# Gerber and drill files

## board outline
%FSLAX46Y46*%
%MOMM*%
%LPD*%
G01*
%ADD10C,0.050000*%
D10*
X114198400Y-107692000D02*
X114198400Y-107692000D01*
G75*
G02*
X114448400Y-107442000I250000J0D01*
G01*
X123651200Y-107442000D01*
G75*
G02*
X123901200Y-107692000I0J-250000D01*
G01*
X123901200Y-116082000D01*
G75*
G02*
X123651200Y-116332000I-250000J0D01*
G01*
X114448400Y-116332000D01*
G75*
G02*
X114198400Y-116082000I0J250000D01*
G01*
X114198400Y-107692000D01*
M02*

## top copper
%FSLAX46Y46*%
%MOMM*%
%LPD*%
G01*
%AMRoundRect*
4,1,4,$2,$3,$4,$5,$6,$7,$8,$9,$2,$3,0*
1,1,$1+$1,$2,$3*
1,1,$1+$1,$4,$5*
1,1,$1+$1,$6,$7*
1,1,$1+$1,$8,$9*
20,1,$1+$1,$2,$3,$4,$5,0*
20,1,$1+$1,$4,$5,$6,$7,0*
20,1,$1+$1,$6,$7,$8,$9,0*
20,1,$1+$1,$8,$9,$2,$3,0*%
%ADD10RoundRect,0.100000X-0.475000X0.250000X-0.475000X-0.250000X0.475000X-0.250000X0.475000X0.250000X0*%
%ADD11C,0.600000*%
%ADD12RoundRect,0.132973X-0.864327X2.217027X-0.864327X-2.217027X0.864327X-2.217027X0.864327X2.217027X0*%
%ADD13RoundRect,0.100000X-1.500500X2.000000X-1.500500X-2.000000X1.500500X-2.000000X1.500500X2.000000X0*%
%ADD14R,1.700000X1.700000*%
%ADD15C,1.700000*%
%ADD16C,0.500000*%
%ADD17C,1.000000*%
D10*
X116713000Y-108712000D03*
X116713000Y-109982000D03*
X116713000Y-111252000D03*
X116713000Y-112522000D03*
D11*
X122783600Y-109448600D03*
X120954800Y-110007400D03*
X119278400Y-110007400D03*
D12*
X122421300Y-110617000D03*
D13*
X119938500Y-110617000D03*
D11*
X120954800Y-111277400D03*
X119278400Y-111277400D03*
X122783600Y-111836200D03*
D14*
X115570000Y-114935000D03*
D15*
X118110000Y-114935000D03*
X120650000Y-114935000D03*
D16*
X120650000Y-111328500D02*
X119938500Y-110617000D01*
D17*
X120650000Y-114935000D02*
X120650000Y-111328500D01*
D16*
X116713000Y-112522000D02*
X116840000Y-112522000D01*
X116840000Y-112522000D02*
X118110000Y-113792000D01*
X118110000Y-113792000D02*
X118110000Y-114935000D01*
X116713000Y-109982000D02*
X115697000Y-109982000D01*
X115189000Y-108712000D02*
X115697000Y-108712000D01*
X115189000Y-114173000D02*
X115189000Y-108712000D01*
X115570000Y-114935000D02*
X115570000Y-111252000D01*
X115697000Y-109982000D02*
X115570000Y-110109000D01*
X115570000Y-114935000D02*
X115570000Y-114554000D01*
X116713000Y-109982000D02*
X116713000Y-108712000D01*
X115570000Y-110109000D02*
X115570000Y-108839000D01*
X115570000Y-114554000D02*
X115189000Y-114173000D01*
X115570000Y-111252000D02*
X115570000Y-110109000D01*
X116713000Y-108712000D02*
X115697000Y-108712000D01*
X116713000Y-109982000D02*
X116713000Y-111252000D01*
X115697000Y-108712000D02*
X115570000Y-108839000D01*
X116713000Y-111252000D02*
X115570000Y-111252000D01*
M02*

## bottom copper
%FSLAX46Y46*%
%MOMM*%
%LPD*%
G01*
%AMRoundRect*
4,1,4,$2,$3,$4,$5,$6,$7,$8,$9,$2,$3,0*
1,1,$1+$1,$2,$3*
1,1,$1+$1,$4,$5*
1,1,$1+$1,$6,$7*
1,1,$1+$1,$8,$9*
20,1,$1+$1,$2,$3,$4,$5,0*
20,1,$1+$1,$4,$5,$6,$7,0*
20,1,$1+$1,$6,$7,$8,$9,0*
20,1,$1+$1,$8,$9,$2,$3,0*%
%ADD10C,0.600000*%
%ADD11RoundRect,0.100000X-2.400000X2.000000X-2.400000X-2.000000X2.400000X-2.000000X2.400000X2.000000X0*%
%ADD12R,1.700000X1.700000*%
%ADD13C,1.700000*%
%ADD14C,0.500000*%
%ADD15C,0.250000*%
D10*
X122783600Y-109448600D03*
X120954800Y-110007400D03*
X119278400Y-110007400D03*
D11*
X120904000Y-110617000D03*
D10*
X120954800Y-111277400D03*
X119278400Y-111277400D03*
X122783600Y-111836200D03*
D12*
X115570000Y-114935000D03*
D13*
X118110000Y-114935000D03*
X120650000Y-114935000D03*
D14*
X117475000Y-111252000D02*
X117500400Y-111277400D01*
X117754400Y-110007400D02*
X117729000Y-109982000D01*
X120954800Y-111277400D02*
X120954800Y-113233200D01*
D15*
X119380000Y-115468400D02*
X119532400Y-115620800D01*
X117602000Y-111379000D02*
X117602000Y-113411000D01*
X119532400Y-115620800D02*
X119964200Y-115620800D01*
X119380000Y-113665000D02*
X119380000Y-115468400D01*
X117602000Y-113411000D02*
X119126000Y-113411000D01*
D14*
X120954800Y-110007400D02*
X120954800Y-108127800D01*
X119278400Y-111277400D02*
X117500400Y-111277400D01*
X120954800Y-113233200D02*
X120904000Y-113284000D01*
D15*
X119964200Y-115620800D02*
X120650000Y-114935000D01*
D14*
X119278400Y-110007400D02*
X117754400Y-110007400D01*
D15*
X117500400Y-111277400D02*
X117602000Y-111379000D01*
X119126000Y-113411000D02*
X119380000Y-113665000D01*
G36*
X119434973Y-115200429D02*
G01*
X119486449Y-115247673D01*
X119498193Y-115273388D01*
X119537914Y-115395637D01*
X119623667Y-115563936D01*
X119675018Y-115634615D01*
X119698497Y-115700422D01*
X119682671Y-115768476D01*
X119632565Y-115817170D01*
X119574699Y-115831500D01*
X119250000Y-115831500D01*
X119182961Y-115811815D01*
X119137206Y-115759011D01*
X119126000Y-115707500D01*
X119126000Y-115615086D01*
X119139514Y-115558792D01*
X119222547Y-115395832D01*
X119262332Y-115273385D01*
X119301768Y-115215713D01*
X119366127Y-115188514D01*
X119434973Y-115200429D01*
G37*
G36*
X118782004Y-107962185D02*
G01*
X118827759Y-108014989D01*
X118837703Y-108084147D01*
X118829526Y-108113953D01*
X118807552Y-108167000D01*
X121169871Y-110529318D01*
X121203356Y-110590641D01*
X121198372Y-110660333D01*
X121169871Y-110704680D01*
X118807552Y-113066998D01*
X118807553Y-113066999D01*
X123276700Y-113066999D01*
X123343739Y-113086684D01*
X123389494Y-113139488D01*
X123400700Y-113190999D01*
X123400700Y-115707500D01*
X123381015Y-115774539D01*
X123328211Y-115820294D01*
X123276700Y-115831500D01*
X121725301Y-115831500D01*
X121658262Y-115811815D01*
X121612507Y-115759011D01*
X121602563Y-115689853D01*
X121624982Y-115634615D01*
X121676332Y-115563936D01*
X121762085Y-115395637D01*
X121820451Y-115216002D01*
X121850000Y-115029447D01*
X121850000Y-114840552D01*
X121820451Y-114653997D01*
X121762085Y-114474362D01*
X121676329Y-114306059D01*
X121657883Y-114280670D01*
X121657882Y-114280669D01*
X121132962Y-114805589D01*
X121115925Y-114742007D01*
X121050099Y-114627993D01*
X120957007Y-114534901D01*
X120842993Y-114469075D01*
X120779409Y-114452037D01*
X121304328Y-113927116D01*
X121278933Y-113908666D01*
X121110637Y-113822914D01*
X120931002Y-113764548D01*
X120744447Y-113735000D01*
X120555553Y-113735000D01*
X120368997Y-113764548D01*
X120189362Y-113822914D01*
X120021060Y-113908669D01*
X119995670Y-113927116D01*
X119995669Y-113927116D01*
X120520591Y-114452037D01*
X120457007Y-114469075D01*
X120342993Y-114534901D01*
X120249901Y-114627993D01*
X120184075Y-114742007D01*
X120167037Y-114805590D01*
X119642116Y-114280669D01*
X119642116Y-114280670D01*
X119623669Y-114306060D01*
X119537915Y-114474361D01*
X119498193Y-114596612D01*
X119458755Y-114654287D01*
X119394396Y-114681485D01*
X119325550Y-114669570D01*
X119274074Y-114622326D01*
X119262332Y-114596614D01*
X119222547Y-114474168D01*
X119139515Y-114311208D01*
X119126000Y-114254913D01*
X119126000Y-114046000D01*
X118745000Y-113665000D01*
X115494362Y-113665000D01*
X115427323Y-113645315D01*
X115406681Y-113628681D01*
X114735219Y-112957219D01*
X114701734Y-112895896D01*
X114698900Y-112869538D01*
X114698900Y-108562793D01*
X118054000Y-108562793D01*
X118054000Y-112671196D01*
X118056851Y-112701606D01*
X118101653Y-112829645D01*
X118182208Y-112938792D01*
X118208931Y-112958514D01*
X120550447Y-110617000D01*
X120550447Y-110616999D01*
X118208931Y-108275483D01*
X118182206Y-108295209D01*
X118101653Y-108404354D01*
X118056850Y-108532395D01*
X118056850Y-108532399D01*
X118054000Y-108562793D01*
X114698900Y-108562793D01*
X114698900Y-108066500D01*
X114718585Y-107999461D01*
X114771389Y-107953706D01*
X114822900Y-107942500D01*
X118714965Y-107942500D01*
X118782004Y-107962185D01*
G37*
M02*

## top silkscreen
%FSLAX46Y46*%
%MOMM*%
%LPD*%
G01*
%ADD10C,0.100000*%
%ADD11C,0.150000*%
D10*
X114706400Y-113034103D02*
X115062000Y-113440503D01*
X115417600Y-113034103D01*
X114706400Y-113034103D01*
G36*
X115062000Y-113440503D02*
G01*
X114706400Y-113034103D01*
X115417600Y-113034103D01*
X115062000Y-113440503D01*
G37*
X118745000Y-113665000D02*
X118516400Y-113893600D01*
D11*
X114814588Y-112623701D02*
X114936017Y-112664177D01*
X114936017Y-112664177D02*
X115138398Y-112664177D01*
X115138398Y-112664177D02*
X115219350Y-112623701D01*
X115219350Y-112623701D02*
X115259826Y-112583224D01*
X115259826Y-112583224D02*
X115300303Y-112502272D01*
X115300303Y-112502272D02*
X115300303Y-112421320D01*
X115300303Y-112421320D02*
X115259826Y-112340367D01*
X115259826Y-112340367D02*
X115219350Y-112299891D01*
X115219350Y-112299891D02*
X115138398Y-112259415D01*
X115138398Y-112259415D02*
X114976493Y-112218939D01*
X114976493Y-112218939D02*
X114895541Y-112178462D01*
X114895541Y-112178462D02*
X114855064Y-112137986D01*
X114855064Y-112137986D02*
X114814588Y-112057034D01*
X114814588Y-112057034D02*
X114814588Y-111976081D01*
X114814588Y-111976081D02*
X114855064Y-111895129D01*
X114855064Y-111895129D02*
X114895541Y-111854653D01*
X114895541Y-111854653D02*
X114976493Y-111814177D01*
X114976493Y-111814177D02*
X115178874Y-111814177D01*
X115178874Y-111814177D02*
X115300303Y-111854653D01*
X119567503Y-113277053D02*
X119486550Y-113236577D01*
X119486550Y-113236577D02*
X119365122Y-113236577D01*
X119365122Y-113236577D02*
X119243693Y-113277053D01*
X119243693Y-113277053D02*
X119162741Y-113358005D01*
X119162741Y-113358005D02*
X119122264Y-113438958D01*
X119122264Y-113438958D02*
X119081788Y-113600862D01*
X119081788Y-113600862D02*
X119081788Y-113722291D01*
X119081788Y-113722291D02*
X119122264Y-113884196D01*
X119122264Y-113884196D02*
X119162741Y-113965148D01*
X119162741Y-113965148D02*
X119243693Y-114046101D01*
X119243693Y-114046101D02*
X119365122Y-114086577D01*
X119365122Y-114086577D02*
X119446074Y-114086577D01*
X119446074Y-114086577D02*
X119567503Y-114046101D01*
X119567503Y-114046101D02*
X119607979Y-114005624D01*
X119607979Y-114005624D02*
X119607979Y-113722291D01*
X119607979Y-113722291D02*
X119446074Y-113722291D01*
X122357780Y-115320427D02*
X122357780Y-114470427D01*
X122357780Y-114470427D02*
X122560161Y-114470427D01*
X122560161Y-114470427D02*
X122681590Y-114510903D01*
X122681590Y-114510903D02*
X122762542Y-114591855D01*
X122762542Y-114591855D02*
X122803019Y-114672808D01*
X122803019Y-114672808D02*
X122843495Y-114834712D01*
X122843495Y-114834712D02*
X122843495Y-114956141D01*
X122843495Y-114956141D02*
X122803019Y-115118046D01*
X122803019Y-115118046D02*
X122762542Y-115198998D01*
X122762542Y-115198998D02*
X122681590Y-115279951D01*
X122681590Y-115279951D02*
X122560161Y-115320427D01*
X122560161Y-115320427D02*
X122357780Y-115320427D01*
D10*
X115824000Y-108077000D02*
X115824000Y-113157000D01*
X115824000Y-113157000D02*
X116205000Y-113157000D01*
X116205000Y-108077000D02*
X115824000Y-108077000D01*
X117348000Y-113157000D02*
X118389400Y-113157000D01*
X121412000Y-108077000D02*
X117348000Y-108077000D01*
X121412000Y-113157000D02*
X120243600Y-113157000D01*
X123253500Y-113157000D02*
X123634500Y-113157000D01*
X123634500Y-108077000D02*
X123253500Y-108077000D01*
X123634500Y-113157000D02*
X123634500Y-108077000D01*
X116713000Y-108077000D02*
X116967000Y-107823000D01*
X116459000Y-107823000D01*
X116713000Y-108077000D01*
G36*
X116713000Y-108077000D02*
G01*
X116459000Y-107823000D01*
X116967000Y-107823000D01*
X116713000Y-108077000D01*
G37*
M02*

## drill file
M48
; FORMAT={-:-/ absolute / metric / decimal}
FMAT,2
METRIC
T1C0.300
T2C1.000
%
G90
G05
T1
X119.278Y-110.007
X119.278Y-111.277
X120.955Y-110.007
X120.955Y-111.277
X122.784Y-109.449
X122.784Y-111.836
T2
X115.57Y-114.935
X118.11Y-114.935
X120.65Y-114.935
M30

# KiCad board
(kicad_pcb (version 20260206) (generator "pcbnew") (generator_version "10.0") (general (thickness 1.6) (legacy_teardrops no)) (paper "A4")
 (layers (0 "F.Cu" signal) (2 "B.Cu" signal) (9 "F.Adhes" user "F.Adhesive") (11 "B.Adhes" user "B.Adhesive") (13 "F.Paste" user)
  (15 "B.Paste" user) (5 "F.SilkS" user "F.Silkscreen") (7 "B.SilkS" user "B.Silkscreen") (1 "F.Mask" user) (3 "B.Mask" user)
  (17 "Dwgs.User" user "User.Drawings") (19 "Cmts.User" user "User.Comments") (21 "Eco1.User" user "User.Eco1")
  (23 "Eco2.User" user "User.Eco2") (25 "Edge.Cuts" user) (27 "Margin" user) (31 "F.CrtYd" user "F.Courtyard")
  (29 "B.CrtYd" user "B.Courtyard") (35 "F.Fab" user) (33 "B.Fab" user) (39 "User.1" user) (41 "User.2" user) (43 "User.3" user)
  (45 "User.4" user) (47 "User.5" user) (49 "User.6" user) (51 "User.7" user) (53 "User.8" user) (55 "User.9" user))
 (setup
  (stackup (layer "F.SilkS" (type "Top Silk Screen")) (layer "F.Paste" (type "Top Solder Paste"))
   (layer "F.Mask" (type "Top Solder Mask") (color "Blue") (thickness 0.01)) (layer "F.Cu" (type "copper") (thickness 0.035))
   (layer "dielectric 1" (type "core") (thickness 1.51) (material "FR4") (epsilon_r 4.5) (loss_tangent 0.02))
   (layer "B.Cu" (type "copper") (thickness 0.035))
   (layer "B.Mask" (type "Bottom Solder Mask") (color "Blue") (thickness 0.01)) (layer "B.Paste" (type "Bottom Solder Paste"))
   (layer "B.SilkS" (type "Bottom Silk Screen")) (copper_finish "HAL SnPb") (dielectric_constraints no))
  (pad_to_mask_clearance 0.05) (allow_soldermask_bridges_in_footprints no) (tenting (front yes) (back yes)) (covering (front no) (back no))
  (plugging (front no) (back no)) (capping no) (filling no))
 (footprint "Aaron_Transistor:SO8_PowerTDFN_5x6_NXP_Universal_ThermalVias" (layer "F.Cu") (at 122.936 110.617 -90)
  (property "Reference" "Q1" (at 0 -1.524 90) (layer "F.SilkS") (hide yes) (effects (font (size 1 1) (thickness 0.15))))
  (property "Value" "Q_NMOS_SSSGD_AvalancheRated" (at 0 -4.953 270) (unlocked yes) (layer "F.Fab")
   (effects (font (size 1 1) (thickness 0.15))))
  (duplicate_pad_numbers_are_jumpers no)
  (fp_line (start -2.54 7.112) (end 2.54 7.112) (stroke (width 0.1) (type default)) (layer "F.SilkS"))
  (fp_line (start 2.54 7.112) (end 2.54 6.731) (stroke (width 0.1) (type default)) (layer "F.SilkS"))
  (fp_line (start -2.54 6.731) (end -2.54 7.112) (stroke (width 0.1) (type default)) (layer "F.SilkS"))
  (fp_line (start 2.54 5.588) (end 2.54 4.5466) (stroke (width 0.1) (type default)) (layer "F.SilkS"))
  (fp_line (start -2.54 1.524) (end -2.54 5.588) (stroke (width 0.1) (type default)) (layer "F.SilkS"))
  (fp_line (start 2.54 1.524) (end 2.54 2.6924) (stroke (width 0.1) (type default)) (layer "F.SilkS"))
  (fp_line (start 2.54 -0.3175) (end 2.54 -0.6985) (stroke (width 0.1) (type default)) (layer "F.SilkS"))
  (fp_line (start -2.54 -0.6985) (end -2.54 -0.3175) (stroke (width 0.1) (type default)) (layer "F.SilkS"))
  (fp_line (start 2.54 -0.6985) (end -2.54 -0.6985) (stroke (width 0.1) (type default)) (layer "F.SilkS"))
  (fp_poly (pts (xy -2.54 6.223) (xy -2.794 5.969) (xy -2.794 6.477)) (stroke (width 0.1) (type solid)) (fill yes) (layer "F.SilkS"))
  (pad "1" smd roundrect (at -1.905 6.223 270) (size 0.7 1.15) (layers "F.Cu" "F.Mask" "F.Paste") (roundrect_rratio 0.1428571429)
   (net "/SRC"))
  (pad "2" smd roundrect (at -0.635 6.223 270) (size 0.7 1.15) (layers "F.Cu" "F.Mask" "F.Paste") (roundrect_rratio 0.1428571429)
   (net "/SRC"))
  (pad "3" smd roundrect (at 0.635 6.223 270) (size 0.7 1.15) (layers "F.Cu" "F.Mask" "F.Paste") (roundrect_rratio 0.1428571429)
   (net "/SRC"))
  (pad "4" smd roundrect (at 1.905 6.223 270) (size 0.7 1.15) (layers "F.Cu" "F.Mask" "F.Paste") (roundrect_rratio 0.1428571429)
   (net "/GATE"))
  (pad "5" thru_hole circle (at -1.1684 0.1524 270) (size 0.6 0.6) (drill 0.3) (layers "*.Cu" "*.Mask") (remove_unused_layers no)
   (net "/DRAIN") (zone_connect 2))
  (pad "5" thru_hole circle (at -0.6096 1.9812 270) (size 0.6 0.6) (drill 0.3) (layers "*.Cu" "*.Mask") (remove_unused_layers no)
   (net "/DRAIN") (zone_connect 2))
  (pad "5" thru_hole circle (at -0.6096 3.6576 270) (size 0.6 0.6) (drill 0.3) (layers "*.Cu" "*.Mask") (remove_unused_layers no)
   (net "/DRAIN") (zone_connect 2))
  (pad "5" smd roundrect (at 0 0.5147 270) (size 4.7 1.9946) (layers "F.Cu" "F.Mask") (roundrect_rratio 0.06666666667) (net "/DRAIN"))
  (pad "5" smd roundrect (at 0 2.032 270) (size 4.2 5) (layers "B.Cu" "B.Mask") (roundrect_rratio 0.02380952381) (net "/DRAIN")
   (thermal_bridge_angle 45))
  (pad "5" smd roundrect (at 0 2.9975 270) (size 4.2 3.201) (layers "F.Cu" "F.Mask") (roundrect_rratio 0.03124023743) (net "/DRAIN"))
  (pad "5" thru_hole circle (at 0.6604 1.9812 270) (size 0.6 0.6) (drill 0.3) (layers "*.Cu" "*.Mask") (remove_unused_layers no)
   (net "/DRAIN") (zone_connect 2))
  (pad "5" thru_hole circle (at 0.6604 3.6576 270) (size 0.6 0.6) (drill 0.3) (layers "*.Cu" "*.Mask") (remove_unused_layers no)
   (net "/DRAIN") (zone_connect 2))
  (pad "5" thru_hole circle (at 1.2192 0.1524 270) (size 0.6 0.6) (drill 0.3) (layers "*.Cu" "*.Mask") (remove_unused_layers no)
   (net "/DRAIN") (zone_connect 2)))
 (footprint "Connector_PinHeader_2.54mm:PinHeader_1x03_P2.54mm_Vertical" (layer "B.Cu") (at 115.57 114.935 -90)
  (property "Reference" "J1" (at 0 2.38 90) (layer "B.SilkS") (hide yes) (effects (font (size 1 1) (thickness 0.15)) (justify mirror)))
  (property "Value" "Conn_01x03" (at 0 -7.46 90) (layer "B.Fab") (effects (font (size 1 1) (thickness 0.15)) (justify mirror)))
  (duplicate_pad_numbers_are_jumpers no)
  (pad "1" thru_hole rect (at 0 0 270) (size 1.7 1.7) (drill 1) (layers "*.Cu" "*.Mask") (remove_unused_layers no) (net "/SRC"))
  (pad "2" thru_hole circle (at 0 -2.54 270) (size 1.7 1.7) (drill 1) (layers "*.Cu" "*.Mask") (remove_unused_layers no) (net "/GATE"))
  (pad "3" thru_hole circle (at 0 -5.08 270) (size 1.7 1.7) (drill 1) (layers "*.Cu" "*.Mask") (remove_unused_layers no) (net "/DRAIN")))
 (gr_poly
  (pts (xy 114.7064 113.034103) (xy 115.062 113.440503) (xy 115.4176 113.034103)) (stroke (width 0.1) (type solid)) (fill yes)
  (layer "F.SilkS"))
 (gr_line (start 118.745 113.665) (end 118.5164 113.8936) (stroke (width 0.1) (type default)) (layer "F.SilkS"))
 (gr_rect (start 114.1984 107.442) (end 123.9012 116.332) (radius 0.25) (stroke (width 0.05) (type solid)) (fill no) (layer "Edge.Cuts"))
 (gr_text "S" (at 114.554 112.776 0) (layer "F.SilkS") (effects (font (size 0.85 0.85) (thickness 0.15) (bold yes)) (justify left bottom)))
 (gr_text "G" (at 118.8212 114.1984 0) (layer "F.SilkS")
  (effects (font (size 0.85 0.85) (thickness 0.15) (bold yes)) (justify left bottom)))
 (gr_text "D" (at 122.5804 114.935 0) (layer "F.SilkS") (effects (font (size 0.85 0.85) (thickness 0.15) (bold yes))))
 (segment (start 120.65 111.3285) (end 119.9385 110.617) (width 0.5) (layer "F.Cu") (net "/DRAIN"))
 (segment (start 120.65 114.935) (end 120.65 111.3285) (width 1) (layer "F.Cu") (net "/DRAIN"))
 (segment (start 117.475 111.252) (end 117.5004 111.2774) (width 0.5) (layer "B.Cu") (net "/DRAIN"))
 (segment (start 117.7544 110.0074) (end 117.729 109.982) (width 0.5) (layer "B.Cu") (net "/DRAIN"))
 (segment (start 120.9548 111.2774) (end 120.9548 113.2332) (width 0.5) (layer "B.Cu") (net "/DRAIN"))
 (segment (start 119.38 115.4684) (end 119.5324 115.6208) (width 0.25) (layer "B.Cu") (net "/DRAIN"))
 (segment (start 117.602 111.379) (end 117.602 113.411) (width 0.25) (layer "B.Cu") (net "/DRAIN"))
 (segment (start 119.5324 115.6208) (end 119.9642 115.6208) (width 0.25) (layer "B.Cu") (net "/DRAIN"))
 (segment (start 119.38 113.665) (end 119.38 115.4684) (width 0.25) (layer "B.Cu") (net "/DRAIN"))
 (segment (start 117.602 113.411) (end 119.126 113.411) (width 0.25) (layer "B.Cu") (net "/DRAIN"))
 (segment (start 120.9548 110.0074) (end 120.9548 108.1278) (width 0.5) (layer "B.Cu") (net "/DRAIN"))
 (segment (start 119.2784 111.2774) (end 117.5004 111.2774) (width 0.5) (layer "B.Cu") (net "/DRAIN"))
 (segment (start 120.9548 113.2332) (end 120.904 113.284) (width 0.5) (layer "B.Cu") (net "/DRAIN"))
 (segment (start 119.9642 115.6208) (end 120.65 114.935) (width 0.25) (layer "B.Cu") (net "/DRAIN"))
 (segment (start 119.2784 110.0074) (end 117.7544 110.0074) (width 0.5) (layer "B.Cu") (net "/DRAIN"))
 (segment (start 117.5004 111.2774) (end 117.602 111.379) (width 0.25) (layer "B.Cu") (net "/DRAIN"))
 (segment (start 119.126 113.411) (end 119.38 113.665) (width 0.25) (layer "B.Cu") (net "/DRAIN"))
 (segment (start 116.713 112.522) (end 116.84 112.522) (width 0.5) (layer "F.Cu") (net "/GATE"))
 (segment (start 116.84 112.522) (end 118.11 113.792) (width 0.5) (layer "F.Cu") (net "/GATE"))
 (segment (start 118.11 113.792) (end 118.11 114.935) (width 0.5) (layer "F.Cu") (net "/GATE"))
 (segment (start 116.713 109.982) (end 115.697 109.982) (width 0.5) (layer "F.Cu") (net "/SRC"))
 (segment (start 115.189 108.712) (end 115.697 108.712) (width 0.5) (layer "F.Cu") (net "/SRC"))
 (segment (start 115.189 114.173) (end 115.189 108.712) (width 0.5) (layer "F.Cu") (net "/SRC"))
 (segment (start 115.57 114.935) (end 115.57 111.252) (width 0.5) (layer "F.Cu") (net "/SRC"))
 (segment (start 115.697 109.982) (end 115.57 110.109) (width 0.5) (layer "F.Cu") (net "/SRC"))
 (segment (start 115.57 114.935) (end 115.57 114.554) (width 0.5) (layer "F.Cu") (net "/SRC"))
 (segment (start 116.713 109.982) (end 116.713 108.712) (width 0.5) (layer "F.Cu") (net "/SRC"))
 (segment (start 115.57 110.109) (end 115.57 108.839) (width 0.5) (layer "F.Cu") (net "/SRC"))
 (segment (start 115.57 114.554) (end 115.189 114.173) (width 0.5) (layer "F.Cu") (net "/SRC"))
 (segment (start 115.57 111.252) (end 115.57 110.109) (width 0.5) (layer "F.Cu") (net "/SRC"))
 (segment (start 116.713 108.712) (end 115.697 108.712) (width 0.5) (layer "F.Cu") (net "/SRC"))
 (segment (start 116.713 109.982) (end 116.713 111.252) (width 0.5) (layer "F.Cu") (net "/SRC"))
 (segment (start 115.697 108.712) (end 115.57 108.839) (width 0.5) (layer "F.Cu") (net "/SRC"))
 (segment (start 116.713 111.252) (end 115.57 111.252) (width 0.5) (layer "F.Cu") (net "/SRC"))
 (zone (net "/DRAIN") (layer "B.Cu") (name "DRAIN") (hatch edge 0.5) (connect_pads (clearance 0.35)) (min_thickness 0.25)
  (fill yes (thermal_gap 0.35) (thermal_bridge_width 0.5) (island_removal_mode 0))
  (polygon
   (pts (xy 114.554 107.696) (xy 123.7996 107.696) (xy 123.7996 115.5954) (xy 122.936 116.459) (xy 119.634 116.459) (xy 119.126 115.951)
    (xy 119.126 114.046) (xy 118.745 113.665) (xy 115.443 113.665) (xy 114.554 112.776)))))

